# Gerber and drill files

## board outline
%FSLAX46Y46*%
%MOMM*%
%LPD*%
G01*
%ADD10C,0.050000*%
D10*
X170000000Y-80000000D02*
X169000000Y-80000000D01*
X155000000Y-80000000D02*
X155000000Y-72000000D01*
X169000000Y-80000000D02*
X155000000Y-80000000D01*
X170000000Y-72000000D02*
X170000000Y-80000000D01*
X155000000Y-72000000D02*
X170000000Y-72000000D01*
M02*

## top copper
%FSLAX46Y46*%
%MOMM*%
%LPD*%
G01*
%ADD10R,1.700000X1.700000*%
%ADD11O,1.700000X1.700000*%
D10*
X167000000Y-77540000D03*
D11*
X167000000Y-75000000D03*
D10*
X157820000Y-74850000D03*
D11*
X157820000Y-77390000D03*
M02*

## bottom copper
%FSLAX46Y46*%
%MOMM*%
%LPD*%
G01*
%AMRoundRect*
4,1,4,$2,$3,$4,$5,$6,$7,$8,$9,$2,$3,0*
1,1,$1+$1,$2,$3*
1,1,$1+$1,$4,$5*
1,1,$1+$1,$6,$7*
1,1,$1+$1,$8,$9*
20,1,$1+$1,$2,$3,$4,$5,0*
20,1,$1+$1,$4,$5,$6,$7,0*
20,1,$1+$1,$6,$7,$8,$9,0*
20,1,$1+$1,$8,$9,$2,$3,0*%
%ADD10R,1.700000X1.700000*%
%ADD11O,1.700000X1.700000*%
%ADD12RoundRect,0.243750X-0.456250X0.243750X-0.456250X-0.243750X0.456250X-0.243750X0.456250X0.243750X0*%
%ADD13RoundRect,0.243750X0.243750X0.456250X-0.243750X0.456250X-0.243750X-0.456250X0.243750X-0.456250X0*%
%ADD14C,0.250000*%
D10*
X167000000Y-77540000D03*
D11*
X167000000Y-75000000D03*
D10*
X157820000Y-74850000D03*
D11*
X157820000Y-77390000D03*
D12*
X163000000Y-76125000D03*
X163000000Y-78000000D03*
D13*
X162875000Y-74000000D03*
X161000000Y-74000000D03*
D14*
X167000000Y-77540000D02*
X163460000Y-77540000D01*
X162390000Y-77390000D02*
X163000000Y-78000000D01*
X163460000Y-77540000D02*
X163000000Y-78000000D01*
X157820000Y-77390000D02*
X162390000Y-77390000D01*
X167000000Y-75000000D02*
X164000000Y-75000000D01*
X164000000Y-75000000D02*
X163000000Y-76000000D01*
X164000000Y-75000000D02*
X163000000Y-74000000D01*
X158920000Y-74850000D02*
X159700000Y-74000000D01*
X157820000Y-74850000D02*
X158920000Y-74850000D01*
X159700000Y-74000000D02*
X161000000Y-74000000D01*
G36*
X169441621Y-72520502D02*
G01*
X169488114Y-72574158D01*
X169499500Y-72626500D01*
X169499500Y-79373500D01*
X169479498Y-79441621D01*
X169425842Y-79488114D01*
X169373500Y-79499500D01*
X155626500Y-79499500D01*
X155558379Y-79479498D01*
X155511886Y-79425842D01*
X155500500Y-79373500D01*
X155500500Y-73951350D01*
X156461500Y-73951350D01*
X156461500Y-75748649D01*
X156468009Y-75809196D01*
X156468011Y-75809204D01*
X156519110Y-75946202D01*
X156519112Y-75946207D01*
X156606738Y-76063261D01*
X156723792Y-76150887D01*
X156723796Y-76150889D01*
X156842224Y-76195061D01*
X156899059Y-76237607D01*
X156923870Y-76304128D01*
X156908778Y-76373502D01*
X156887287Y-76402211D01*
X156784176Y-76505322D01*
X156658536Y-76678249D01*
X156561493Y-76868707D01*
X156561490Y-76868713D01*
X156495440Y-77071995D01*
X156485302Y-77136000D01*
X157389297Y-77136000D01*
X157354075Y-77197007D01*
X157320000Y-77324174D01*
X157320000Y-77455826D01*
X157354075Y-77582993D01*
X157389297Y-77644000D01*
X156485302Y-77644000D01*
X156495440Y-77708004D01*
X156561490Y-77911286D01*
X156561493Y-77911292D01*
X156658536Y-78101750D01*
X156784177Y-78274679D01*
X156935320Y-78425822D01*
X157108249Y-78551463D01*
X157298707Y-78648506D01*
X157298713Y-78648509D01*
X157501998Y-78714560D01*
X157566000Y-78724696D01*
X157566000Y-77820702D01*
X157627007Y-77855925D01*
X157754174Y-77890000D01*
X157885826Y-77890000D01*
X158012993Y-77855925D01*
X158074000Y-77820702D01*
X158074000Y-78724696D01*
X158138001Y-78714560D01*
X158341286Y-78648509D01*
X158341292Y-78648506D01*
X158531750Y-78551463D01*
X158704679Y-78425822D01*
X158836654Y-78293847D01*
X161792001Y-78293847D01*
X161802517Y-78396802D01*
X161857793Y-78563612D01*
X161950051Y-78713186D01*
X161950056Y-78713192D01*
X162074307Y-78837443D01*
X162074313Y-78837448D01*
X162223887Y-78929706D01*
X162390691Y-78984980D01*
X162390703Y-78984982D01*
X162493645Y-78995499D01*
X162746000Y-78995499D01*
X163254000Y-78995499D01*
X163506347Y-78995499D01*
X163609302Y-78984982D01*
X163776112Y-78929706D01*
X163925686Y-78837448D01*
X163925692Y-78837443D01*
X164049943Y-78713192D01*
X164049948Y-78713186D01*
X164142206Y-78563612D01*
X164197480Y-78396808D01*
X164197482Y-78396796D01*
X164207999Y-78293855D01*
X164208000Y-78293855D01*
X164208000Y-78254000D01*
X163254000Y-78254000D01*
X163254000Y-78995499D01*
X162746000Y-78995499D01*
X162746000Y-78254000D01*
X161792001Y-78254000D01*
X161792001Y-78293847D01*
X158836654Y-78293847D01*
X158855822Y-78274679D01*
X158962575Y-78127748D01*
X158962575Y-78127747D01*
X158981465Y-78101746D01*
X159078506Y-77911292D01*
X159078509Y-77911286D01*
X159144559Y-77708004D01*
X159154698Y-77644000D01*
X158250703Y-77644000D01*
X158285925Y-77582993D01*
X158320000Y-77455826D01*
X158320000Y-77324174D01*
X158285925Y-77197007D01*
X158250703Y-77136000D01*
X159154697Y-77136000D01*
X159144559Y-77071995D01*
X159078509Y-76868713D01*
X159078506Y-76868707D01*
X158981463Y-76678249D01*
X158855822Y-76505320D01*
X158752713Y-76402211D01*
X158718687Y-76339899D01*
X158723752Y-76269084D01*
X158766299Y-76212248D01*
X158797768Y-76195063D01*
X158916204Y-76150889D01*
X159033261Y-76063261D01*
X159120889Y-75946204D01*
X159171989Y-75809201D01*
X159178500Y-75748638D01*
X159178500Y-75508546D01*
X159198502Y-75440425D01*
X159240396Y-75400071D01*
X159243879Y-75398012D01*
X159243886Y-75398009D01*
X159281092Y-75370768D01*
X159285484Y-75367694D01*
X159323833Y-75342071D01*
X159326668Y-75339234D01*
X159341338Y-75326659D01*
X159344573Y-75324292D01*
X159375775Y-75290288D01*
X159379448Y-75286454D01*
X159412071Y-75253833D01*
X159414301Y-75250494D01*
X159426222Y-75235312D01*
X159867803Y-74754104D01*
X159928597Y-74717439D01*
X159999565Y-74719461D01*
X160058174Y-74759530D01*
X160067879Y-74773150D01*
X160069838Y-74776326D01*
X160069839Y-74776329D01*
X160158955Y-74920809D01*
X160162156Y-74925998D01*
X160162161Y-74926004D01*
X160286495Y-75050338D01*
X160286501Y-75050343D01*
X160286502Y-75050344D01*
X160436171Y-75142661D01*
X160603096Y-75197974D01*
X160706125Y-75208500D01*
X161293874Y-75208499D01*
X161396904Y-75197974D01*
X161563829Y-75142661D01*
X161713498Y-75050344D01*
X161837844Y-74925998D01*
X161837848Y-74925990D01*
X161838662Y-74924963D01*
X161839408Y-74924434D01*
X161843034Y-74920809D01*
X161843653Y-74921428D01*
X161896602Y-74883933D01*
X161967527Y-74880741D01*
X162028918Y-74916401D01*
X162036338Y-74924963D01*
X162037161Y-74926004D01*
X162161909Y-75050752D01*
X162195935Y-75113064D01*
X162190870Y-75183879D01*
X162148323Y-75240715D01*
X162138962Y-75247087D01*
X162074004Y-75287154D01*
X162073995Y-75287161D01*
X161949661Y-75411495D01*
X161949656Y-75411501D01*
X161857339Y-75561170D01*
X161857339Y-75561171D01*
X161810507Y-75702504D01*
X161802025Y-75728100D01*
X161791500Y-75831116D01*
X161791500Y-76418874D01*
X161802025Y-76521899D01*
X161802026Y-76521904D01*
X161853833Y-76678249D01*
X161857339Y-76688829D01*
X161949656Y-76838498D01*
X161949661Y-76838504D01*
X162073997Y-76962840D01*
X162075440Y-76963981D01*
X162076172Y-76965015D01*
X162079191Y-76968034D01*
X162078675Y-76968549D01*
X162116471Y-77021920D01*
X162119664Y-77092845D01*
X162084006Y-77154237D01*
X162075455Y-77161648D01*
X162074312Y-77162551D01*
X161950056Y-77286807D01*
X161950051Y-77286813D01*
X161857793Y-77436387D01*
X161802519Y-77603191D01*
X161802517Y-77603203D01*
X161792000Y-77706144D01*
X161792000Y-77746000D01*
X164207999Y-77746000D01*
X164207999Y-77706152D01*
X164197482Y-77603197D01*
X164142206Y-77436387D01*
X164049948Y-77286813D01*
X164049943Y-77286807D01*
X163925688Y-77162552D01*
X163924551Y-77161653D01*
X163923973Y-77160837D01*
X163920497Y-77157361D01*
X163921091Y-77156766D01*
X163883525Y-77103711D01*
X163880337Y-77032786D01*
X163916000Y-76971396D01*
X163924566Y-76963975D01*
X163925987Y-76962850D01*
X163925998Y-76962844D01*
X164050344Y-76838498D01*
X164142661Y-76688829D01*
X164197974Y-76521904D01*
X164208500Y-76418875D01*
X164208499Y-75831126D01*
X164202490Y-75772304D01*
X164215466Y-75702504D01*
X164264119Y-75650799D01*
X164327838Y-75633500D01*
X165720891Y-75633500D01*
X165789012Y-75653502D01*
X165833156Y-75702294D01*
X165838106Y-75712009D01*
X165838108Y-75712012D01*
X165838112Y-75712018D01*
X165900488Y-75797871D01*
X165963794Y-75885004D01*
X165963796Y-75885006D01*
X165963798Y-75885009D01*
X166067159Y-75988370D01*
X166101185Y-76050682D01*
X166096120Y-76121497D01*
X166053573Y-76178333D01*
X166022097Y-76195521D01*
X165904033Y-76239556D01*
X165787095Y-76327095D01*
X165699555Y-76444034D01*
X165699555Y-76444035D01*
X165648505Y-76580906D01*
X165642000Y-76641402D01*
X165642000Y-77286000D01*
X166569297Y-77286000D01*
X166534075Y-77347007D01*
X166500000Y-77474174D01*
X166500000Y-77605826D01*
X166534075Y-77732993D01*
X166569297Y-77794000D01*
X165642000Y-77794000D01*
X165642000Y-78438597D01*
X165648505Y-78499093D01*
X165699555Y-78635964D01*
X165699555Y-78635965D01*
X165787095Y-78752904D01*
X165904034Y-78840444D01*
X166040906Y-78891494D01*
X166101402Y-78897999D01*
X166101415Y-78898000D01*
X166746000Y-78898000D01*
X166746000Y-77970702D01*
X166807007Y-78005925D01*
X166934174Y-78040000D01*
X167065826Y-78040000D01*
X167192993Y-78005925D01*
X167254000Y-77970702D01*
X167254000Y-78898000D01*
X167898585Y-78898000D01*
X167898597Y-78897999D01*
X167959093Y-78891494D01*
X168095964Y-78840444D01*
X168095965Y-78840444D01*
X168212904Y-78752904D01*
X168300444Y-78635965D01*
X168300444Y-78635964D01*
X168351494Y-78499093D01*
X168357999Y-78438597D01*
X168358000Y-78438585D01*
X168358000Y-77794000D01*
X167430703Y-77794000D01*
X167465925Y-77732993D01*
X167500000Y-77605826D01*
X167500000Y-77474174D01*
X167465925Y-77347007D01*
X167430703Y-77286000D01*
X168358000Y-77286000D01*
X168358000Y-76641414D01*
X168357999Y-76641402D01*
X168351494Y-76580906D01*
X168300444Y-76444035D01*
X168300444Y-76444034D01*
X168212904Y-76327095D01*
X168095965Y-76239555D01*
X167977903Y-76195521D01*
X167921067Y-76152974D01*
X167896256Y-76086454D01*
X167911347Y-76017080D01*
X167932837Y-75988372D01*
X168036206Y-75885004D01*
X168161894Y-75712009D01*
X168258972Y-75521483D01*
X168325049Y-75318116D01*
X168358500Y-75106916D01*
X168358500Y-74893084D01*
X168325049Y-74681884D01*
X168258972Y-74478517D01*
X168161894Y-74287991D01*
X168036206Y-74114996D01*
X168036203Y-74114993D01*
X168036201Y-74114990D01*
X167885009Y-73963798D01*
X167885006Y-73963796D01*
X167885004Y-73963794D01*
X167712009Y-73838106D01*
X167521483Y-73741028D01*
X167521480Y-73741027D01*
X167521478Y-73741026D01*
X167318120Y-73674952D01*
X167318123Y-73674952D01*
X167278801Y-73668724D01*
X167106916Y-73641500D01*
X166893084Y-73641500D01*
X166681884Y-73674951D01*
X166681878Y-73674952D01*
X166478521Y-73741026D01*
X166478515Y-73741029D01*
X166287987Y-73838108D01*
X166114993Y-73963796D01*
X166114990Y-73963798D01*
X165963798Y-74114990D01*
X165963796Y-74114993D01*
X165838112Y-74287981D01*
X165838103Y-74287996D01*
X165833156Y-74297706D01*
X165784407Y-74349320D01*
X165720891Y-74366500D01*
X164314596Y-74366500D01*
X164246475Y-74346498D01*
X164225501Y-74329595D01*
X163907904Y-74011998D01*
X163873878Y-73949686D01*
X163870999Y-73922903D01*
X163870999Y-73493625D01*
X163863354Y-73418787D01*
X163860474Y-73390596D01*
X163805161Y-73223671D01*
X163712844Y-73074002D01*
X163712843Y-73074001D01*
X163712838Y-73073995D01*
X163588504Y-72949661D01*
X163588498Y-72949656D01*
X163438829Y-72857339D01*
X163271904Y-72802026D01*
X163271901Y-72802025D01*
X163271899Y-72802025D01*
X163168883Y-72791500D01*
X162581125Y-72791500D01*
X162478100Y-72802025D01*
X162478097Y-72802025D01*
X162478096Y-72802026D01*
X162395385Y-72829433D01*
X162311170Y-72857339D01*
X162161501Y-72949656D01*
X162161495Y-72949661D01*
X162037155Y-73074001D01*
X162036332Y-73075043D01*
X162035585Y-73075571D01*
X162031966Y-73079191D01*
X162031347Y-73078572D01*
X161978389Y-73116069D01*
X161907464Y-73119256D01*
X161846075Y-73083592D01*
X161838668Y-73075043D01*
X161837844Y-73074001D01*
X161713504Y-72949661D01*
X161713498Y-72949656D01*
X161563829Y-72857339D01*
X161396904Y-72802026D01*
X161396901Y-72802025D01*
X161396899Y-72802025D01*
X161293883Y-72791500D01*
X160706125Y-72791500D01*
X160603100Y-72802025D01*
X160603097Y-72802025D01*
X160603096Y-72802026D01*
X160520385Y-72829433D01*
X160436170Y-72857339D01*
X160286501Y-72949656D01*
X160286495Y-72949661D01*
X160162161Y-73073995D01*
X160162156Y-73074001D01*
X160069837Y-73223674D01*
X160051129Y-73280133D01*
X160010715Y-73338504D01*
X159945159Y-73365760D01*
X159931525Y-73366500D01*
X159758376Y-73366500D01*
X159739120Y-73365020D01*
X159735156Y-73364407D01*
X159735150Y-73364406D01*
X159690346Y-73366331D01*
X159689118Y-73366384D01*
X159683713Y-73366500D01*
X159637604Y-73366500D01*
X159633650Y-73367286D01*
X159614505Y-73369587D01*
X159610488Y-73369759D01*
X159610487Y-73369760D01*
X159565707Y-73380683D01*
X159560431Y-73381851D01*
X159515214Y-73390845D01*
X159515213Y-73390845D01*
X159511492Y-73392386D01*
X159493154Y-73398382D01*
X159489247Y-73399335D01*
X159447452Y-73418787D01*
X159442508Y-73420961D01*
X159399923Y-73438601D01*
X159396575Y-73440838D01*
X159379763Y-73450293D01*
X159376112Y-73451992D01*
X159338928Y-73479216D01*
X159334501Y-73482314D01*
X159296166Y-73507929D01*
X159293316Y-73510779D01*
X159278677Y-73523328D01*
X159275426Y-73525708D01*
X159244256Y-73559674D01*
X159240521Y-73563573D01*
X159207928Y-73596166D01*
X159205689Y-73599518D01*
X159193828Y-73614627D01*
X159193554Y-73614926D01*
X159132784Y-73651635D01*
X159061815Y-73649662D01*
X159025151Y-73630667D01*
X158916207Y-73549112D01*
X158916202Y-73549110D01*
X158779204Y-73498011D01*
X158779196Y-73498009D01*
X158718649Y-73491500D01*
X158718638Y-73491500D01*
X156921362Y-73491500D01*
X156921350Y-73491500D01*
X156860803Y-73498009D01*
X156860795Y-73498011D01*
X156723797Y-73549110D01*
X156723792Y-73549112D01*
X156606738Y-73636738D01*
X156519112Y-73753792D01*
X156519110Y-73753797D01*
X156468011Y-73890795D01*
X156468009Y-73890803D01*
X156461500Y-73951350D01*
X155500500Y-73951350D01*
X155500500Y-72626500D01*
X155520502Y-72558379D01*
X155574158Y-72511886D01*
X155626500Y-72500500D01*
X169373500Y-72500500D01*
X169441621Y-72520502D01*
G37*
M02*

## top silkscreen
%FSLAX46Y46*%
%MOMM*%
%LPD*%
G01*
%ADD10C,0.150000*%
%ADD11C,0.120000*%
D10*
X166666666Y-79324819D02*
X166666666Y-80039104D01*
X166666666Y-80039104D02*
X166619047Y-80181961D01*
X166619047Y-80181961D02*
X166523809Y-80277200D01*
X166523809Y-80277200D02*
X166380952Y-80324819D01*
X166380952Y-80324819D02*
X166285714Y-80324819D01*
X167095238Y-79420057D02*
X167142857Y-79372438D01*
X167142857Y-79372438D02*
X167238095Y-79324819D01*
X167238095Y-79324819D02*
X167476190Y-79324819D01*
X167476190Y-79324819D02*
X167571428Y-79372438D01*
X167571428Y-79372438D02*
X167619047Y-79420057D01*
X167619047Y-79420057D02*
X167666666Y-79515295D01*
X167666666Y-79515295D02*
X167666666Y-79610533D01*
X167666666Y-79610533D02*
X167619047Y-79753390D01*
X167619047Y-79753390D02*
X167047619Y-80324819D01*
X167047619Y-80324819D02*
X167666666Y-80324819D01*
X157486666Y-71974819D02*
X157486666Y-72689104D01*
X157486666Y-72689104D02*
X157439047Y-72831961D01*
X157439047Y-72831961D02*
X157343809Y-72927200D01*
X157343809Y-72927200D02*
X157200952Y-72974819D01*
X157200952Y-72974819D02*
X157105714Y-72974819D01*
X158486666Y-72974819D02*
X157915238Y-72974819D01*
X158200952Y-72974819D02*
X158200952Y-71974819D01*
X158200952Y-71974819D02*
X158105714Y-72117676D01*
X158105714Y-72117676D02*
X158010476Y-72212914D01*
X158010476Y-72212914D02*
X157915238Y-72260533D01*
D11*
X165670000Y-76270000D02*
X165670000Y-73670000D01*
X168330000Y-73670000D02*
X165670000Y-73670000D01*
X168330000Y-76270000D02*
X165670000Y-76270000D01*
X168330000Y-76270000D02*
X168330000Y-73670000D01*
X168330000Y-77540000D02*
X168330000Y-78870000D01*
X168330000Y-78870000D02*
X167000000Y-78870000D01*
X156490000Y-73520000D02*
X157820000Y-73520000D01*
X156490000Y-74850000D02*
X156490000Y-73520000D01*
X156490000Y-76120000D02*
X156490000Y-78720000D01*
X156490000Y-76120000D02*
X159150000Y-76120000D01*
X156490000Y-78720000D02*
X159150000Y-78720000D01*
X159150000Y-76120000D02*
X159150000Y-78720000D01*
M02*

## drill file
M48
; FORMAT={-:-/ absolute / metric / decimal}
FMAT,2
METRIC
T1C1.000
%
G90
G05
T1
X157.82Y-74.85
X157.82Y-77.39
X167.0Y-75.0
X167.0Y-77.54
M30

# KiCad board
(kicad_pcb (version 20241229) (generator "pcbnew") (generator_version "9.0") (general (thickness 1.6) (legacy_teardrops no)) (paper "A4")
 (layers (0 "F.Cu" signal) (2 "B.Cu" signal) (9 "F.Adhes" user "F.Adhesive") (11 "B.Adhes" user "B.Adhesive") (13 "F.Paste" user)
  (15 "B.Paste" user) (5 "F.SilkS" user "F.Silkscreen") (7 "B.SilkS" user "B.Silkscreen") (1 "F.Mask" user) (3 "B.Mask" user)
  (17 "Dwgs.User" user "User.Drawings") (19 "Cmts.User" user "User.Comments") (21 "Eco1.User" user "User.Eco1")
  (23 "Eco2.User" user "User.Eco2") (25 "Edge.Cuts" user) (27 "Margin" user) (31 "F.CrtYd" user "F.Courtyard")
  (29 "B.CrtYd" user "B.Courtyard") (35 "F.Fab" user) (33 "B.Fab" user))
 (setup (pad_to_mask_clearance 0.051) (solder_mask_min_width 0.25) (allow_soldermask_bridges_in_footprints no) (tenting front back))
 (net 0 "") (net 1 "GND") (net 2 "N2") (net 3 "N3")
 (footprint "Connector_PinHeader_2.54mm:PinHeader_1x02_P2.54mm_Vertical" (layer "F.Cu") (at 167 77.54 180)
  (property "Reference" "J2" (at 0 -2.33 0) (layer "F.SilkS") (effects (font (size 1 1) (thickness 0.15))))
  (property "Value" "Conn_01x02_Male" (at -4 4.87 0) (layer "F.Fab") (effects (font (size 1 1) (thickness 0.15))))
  (fp_line (start 1.33 1.27) (end 1.33 3.87) (stroke (width 0.12) (type solid)) (layer "F.SilkS"))
  (fp_line (start -1.33 3.87) (end 1.33 3.87) (stroke (width 0.12) (type solid)) (layer "F.SilkS"))
  (fp_line (start -1.33 1.27) (end 1.33 1.27) (stroke (width 0.12) (type solid)) (layer "F.SilkS"))
  (fp_line (start -1.33 1.27) (end -1.33 3.87) (stroke (width 0.12) (type solid)) (layer "F.SilkS"))
  (fp_line (start -1.33 0) (end -1.33 -1.33) (stroke (width 0.12) (type solid)) (layer "F.SilkS"))
  (fp_line (start -1.33 -1.33) (end 0 -1.33) (stroke (width 0.12) (type solid)) (layer "F.SilkS"))
  (pad "1" thru_hole rect (at 0 0 180) (size 1.7 1.7) (drill 1) (layers "*.Cu" "*.Mask") (remove_unused_layers no) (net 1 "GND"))
  (pad "2" thru_hole oval (at 0 2.54 180) (size 1.7 1.7) (drill 1) (layers "*.Cu" "*.Mask") (remove_unused_layers no) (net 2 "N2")))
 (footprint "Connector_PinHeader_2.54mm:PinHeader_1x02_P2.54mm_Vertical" (layer "F.Cu") (at 157.82 74.85)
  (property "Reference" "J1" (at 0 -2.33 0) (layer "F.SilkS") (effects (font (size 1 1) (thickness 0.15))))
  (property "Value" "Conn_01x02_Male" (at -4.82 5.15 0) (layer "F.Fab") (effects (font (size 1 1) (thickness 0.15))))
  (fp_line (start -1.33 -1.33) (end 0 -1.33) (stroke (width 0.12) (type solid)) (layer "F.SilkS"))
  (fp_line (start -1.33 0) (end -1.33 -1.33) (stroke (width 0.12) (type solid)) (layer "F.SilkS"))
  (fp_line (start -1.33 1.27) (end -1.33 3.87) (stroke (width 0.12) (type solid)) (layer "F.SilkS"))
  (fp_line (start -1.33 1.27) (end 1.33 1.27) (stroke (width 0.12) (type solid)) (layer "F.SilkS"))
  (fp_line (start -1.33 3.87) (end 1.33 3.87) (stroke (width 0.12) (type solid)) (layer "F.SilkS"))
  (fp_line (start 1.33 1.27) (end 1.33 3.87) (stroke (width 0.12) (type solid)) (layer "F.SilkS"))
  (pad "1" thru_hole rect (at 0 0) (size 1.7 1.7) (drill 1) (layers "*.Cu" "*.Mask") (remove_unused_layers no) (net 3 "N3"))
  (pad "2" thru_hole oval (at 0 2.54) (size 1.7 1.7) (drill 1) (layers "*.Cu" "*.Mask") (remove_unused_layers no) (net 1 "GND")))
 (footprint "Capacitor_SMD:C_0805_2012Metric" (layer "B.Cu") (at 163 77.0625 -90)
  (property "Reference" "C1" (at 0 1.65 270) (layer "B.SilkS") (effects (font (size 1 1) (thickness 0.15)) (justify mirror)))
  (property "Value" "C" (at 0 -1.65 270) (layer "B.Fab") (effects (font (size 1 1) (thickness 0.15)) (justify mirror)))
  (pad "1" smd roundrect (at -0.9375 0 270) (size 0.975 1.4) (layers "B.Cu" "B.Mask" "B.Paste") (roundrect_rratio 0.25) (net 2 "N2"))
  (pad "2" smd roundrect (at 0.9375 0 270) (size 0.975 1.4) (layers "B.Cu" "B.Mask" "B.Paste") (roundrect_rratio 0.25) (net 1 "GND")))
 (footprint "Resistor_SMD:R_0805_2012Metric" (layer "B.Cu") (at 161.9375 74 180)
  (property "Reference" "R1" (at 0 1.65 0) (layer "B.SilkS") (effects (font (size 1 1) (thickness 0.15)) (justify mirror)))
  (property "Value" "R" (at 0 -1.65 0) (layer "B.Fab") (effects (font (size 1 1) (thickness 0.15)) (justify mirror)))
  (pad "1" smd roundrect (at -0.9375 0 180) (size 0.975 1.4) (layers "B.Cu" "B.Mask" "B.Paste") (roundrect_rratio 0.25) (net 2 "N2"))
  (pad "2" smd roundrect (at 0.9375 0 180) (size 0.975 1.4) (layers "B.Cu" "B.Mask" "B.Paste") (roundrect_rratio 0.25) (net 3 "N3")))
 (gr_line (start 170 80) (end 169 80) (stroke (width 0.05) (type solid)) (layer "Edge.Cuts"))
 (gr_line (start 155 80) (end 155 72) (stroke (width 0.05) (type solid)) (layer "Edge.Cuts"))
 (gr_line (start 169 80) (end 155 80) (stroke (width 0.05) (type solid)) (layer "Edge.Cuts"))
 (gr_line (start 170 72) (end 170 80) (stroke (width 0.05) (type solid)) (layer "Edge.Cuts"))
 (gr_line (start 155 72) (end 170 72) (stroke (width 0.05) (type solid)) (layer "Edge.Cuts"))
 (segment (start 167 77.54) (end 163.46 77.54) (width 0.25) (layer "B.Cu") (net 1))
 (segment (start 162.39 77.39) (end 163 78) (width 0.25) (layer "B.Cu") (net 1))
 (segment (start 163.46 77.54) (end 163 78) (width 0.25) (layer "B.Cu") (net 1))
 (segment (start 157.82 77.39) (end 162.39 77.39) (width 0.25) (layer "B.Cu") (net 1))
 (segment (start 167 75) (end 164 75) (width 0.25) (layer "B.Cu") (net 2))
 (segment (start 164 75) (end 163 76) (width 0.25) (layer "B.Cu") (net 2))
 (segment (start 164 75) (end 163 74) (width 0.25) (layer "B.Cu") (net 2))
 (segment (start 158.92 74.85) (end 159.7 74) (width 0.25) (layer "B.Cu") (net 3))
 (segment (start 157.82 74.85) (end 158.92 74.85) (width 0.25) (layer "B.Cu") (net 3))
 (segment (start 159.7 74) (end 161 74) (width 0.25) (layer "B.Cu") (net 3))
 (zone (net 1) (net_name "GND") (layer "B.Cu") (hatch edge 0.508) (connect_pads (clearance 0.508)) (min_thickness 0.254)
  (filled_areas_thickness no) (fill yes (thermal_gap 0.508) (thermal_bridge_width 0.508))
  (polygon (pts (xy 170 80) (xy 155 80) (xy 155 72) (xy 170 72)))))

